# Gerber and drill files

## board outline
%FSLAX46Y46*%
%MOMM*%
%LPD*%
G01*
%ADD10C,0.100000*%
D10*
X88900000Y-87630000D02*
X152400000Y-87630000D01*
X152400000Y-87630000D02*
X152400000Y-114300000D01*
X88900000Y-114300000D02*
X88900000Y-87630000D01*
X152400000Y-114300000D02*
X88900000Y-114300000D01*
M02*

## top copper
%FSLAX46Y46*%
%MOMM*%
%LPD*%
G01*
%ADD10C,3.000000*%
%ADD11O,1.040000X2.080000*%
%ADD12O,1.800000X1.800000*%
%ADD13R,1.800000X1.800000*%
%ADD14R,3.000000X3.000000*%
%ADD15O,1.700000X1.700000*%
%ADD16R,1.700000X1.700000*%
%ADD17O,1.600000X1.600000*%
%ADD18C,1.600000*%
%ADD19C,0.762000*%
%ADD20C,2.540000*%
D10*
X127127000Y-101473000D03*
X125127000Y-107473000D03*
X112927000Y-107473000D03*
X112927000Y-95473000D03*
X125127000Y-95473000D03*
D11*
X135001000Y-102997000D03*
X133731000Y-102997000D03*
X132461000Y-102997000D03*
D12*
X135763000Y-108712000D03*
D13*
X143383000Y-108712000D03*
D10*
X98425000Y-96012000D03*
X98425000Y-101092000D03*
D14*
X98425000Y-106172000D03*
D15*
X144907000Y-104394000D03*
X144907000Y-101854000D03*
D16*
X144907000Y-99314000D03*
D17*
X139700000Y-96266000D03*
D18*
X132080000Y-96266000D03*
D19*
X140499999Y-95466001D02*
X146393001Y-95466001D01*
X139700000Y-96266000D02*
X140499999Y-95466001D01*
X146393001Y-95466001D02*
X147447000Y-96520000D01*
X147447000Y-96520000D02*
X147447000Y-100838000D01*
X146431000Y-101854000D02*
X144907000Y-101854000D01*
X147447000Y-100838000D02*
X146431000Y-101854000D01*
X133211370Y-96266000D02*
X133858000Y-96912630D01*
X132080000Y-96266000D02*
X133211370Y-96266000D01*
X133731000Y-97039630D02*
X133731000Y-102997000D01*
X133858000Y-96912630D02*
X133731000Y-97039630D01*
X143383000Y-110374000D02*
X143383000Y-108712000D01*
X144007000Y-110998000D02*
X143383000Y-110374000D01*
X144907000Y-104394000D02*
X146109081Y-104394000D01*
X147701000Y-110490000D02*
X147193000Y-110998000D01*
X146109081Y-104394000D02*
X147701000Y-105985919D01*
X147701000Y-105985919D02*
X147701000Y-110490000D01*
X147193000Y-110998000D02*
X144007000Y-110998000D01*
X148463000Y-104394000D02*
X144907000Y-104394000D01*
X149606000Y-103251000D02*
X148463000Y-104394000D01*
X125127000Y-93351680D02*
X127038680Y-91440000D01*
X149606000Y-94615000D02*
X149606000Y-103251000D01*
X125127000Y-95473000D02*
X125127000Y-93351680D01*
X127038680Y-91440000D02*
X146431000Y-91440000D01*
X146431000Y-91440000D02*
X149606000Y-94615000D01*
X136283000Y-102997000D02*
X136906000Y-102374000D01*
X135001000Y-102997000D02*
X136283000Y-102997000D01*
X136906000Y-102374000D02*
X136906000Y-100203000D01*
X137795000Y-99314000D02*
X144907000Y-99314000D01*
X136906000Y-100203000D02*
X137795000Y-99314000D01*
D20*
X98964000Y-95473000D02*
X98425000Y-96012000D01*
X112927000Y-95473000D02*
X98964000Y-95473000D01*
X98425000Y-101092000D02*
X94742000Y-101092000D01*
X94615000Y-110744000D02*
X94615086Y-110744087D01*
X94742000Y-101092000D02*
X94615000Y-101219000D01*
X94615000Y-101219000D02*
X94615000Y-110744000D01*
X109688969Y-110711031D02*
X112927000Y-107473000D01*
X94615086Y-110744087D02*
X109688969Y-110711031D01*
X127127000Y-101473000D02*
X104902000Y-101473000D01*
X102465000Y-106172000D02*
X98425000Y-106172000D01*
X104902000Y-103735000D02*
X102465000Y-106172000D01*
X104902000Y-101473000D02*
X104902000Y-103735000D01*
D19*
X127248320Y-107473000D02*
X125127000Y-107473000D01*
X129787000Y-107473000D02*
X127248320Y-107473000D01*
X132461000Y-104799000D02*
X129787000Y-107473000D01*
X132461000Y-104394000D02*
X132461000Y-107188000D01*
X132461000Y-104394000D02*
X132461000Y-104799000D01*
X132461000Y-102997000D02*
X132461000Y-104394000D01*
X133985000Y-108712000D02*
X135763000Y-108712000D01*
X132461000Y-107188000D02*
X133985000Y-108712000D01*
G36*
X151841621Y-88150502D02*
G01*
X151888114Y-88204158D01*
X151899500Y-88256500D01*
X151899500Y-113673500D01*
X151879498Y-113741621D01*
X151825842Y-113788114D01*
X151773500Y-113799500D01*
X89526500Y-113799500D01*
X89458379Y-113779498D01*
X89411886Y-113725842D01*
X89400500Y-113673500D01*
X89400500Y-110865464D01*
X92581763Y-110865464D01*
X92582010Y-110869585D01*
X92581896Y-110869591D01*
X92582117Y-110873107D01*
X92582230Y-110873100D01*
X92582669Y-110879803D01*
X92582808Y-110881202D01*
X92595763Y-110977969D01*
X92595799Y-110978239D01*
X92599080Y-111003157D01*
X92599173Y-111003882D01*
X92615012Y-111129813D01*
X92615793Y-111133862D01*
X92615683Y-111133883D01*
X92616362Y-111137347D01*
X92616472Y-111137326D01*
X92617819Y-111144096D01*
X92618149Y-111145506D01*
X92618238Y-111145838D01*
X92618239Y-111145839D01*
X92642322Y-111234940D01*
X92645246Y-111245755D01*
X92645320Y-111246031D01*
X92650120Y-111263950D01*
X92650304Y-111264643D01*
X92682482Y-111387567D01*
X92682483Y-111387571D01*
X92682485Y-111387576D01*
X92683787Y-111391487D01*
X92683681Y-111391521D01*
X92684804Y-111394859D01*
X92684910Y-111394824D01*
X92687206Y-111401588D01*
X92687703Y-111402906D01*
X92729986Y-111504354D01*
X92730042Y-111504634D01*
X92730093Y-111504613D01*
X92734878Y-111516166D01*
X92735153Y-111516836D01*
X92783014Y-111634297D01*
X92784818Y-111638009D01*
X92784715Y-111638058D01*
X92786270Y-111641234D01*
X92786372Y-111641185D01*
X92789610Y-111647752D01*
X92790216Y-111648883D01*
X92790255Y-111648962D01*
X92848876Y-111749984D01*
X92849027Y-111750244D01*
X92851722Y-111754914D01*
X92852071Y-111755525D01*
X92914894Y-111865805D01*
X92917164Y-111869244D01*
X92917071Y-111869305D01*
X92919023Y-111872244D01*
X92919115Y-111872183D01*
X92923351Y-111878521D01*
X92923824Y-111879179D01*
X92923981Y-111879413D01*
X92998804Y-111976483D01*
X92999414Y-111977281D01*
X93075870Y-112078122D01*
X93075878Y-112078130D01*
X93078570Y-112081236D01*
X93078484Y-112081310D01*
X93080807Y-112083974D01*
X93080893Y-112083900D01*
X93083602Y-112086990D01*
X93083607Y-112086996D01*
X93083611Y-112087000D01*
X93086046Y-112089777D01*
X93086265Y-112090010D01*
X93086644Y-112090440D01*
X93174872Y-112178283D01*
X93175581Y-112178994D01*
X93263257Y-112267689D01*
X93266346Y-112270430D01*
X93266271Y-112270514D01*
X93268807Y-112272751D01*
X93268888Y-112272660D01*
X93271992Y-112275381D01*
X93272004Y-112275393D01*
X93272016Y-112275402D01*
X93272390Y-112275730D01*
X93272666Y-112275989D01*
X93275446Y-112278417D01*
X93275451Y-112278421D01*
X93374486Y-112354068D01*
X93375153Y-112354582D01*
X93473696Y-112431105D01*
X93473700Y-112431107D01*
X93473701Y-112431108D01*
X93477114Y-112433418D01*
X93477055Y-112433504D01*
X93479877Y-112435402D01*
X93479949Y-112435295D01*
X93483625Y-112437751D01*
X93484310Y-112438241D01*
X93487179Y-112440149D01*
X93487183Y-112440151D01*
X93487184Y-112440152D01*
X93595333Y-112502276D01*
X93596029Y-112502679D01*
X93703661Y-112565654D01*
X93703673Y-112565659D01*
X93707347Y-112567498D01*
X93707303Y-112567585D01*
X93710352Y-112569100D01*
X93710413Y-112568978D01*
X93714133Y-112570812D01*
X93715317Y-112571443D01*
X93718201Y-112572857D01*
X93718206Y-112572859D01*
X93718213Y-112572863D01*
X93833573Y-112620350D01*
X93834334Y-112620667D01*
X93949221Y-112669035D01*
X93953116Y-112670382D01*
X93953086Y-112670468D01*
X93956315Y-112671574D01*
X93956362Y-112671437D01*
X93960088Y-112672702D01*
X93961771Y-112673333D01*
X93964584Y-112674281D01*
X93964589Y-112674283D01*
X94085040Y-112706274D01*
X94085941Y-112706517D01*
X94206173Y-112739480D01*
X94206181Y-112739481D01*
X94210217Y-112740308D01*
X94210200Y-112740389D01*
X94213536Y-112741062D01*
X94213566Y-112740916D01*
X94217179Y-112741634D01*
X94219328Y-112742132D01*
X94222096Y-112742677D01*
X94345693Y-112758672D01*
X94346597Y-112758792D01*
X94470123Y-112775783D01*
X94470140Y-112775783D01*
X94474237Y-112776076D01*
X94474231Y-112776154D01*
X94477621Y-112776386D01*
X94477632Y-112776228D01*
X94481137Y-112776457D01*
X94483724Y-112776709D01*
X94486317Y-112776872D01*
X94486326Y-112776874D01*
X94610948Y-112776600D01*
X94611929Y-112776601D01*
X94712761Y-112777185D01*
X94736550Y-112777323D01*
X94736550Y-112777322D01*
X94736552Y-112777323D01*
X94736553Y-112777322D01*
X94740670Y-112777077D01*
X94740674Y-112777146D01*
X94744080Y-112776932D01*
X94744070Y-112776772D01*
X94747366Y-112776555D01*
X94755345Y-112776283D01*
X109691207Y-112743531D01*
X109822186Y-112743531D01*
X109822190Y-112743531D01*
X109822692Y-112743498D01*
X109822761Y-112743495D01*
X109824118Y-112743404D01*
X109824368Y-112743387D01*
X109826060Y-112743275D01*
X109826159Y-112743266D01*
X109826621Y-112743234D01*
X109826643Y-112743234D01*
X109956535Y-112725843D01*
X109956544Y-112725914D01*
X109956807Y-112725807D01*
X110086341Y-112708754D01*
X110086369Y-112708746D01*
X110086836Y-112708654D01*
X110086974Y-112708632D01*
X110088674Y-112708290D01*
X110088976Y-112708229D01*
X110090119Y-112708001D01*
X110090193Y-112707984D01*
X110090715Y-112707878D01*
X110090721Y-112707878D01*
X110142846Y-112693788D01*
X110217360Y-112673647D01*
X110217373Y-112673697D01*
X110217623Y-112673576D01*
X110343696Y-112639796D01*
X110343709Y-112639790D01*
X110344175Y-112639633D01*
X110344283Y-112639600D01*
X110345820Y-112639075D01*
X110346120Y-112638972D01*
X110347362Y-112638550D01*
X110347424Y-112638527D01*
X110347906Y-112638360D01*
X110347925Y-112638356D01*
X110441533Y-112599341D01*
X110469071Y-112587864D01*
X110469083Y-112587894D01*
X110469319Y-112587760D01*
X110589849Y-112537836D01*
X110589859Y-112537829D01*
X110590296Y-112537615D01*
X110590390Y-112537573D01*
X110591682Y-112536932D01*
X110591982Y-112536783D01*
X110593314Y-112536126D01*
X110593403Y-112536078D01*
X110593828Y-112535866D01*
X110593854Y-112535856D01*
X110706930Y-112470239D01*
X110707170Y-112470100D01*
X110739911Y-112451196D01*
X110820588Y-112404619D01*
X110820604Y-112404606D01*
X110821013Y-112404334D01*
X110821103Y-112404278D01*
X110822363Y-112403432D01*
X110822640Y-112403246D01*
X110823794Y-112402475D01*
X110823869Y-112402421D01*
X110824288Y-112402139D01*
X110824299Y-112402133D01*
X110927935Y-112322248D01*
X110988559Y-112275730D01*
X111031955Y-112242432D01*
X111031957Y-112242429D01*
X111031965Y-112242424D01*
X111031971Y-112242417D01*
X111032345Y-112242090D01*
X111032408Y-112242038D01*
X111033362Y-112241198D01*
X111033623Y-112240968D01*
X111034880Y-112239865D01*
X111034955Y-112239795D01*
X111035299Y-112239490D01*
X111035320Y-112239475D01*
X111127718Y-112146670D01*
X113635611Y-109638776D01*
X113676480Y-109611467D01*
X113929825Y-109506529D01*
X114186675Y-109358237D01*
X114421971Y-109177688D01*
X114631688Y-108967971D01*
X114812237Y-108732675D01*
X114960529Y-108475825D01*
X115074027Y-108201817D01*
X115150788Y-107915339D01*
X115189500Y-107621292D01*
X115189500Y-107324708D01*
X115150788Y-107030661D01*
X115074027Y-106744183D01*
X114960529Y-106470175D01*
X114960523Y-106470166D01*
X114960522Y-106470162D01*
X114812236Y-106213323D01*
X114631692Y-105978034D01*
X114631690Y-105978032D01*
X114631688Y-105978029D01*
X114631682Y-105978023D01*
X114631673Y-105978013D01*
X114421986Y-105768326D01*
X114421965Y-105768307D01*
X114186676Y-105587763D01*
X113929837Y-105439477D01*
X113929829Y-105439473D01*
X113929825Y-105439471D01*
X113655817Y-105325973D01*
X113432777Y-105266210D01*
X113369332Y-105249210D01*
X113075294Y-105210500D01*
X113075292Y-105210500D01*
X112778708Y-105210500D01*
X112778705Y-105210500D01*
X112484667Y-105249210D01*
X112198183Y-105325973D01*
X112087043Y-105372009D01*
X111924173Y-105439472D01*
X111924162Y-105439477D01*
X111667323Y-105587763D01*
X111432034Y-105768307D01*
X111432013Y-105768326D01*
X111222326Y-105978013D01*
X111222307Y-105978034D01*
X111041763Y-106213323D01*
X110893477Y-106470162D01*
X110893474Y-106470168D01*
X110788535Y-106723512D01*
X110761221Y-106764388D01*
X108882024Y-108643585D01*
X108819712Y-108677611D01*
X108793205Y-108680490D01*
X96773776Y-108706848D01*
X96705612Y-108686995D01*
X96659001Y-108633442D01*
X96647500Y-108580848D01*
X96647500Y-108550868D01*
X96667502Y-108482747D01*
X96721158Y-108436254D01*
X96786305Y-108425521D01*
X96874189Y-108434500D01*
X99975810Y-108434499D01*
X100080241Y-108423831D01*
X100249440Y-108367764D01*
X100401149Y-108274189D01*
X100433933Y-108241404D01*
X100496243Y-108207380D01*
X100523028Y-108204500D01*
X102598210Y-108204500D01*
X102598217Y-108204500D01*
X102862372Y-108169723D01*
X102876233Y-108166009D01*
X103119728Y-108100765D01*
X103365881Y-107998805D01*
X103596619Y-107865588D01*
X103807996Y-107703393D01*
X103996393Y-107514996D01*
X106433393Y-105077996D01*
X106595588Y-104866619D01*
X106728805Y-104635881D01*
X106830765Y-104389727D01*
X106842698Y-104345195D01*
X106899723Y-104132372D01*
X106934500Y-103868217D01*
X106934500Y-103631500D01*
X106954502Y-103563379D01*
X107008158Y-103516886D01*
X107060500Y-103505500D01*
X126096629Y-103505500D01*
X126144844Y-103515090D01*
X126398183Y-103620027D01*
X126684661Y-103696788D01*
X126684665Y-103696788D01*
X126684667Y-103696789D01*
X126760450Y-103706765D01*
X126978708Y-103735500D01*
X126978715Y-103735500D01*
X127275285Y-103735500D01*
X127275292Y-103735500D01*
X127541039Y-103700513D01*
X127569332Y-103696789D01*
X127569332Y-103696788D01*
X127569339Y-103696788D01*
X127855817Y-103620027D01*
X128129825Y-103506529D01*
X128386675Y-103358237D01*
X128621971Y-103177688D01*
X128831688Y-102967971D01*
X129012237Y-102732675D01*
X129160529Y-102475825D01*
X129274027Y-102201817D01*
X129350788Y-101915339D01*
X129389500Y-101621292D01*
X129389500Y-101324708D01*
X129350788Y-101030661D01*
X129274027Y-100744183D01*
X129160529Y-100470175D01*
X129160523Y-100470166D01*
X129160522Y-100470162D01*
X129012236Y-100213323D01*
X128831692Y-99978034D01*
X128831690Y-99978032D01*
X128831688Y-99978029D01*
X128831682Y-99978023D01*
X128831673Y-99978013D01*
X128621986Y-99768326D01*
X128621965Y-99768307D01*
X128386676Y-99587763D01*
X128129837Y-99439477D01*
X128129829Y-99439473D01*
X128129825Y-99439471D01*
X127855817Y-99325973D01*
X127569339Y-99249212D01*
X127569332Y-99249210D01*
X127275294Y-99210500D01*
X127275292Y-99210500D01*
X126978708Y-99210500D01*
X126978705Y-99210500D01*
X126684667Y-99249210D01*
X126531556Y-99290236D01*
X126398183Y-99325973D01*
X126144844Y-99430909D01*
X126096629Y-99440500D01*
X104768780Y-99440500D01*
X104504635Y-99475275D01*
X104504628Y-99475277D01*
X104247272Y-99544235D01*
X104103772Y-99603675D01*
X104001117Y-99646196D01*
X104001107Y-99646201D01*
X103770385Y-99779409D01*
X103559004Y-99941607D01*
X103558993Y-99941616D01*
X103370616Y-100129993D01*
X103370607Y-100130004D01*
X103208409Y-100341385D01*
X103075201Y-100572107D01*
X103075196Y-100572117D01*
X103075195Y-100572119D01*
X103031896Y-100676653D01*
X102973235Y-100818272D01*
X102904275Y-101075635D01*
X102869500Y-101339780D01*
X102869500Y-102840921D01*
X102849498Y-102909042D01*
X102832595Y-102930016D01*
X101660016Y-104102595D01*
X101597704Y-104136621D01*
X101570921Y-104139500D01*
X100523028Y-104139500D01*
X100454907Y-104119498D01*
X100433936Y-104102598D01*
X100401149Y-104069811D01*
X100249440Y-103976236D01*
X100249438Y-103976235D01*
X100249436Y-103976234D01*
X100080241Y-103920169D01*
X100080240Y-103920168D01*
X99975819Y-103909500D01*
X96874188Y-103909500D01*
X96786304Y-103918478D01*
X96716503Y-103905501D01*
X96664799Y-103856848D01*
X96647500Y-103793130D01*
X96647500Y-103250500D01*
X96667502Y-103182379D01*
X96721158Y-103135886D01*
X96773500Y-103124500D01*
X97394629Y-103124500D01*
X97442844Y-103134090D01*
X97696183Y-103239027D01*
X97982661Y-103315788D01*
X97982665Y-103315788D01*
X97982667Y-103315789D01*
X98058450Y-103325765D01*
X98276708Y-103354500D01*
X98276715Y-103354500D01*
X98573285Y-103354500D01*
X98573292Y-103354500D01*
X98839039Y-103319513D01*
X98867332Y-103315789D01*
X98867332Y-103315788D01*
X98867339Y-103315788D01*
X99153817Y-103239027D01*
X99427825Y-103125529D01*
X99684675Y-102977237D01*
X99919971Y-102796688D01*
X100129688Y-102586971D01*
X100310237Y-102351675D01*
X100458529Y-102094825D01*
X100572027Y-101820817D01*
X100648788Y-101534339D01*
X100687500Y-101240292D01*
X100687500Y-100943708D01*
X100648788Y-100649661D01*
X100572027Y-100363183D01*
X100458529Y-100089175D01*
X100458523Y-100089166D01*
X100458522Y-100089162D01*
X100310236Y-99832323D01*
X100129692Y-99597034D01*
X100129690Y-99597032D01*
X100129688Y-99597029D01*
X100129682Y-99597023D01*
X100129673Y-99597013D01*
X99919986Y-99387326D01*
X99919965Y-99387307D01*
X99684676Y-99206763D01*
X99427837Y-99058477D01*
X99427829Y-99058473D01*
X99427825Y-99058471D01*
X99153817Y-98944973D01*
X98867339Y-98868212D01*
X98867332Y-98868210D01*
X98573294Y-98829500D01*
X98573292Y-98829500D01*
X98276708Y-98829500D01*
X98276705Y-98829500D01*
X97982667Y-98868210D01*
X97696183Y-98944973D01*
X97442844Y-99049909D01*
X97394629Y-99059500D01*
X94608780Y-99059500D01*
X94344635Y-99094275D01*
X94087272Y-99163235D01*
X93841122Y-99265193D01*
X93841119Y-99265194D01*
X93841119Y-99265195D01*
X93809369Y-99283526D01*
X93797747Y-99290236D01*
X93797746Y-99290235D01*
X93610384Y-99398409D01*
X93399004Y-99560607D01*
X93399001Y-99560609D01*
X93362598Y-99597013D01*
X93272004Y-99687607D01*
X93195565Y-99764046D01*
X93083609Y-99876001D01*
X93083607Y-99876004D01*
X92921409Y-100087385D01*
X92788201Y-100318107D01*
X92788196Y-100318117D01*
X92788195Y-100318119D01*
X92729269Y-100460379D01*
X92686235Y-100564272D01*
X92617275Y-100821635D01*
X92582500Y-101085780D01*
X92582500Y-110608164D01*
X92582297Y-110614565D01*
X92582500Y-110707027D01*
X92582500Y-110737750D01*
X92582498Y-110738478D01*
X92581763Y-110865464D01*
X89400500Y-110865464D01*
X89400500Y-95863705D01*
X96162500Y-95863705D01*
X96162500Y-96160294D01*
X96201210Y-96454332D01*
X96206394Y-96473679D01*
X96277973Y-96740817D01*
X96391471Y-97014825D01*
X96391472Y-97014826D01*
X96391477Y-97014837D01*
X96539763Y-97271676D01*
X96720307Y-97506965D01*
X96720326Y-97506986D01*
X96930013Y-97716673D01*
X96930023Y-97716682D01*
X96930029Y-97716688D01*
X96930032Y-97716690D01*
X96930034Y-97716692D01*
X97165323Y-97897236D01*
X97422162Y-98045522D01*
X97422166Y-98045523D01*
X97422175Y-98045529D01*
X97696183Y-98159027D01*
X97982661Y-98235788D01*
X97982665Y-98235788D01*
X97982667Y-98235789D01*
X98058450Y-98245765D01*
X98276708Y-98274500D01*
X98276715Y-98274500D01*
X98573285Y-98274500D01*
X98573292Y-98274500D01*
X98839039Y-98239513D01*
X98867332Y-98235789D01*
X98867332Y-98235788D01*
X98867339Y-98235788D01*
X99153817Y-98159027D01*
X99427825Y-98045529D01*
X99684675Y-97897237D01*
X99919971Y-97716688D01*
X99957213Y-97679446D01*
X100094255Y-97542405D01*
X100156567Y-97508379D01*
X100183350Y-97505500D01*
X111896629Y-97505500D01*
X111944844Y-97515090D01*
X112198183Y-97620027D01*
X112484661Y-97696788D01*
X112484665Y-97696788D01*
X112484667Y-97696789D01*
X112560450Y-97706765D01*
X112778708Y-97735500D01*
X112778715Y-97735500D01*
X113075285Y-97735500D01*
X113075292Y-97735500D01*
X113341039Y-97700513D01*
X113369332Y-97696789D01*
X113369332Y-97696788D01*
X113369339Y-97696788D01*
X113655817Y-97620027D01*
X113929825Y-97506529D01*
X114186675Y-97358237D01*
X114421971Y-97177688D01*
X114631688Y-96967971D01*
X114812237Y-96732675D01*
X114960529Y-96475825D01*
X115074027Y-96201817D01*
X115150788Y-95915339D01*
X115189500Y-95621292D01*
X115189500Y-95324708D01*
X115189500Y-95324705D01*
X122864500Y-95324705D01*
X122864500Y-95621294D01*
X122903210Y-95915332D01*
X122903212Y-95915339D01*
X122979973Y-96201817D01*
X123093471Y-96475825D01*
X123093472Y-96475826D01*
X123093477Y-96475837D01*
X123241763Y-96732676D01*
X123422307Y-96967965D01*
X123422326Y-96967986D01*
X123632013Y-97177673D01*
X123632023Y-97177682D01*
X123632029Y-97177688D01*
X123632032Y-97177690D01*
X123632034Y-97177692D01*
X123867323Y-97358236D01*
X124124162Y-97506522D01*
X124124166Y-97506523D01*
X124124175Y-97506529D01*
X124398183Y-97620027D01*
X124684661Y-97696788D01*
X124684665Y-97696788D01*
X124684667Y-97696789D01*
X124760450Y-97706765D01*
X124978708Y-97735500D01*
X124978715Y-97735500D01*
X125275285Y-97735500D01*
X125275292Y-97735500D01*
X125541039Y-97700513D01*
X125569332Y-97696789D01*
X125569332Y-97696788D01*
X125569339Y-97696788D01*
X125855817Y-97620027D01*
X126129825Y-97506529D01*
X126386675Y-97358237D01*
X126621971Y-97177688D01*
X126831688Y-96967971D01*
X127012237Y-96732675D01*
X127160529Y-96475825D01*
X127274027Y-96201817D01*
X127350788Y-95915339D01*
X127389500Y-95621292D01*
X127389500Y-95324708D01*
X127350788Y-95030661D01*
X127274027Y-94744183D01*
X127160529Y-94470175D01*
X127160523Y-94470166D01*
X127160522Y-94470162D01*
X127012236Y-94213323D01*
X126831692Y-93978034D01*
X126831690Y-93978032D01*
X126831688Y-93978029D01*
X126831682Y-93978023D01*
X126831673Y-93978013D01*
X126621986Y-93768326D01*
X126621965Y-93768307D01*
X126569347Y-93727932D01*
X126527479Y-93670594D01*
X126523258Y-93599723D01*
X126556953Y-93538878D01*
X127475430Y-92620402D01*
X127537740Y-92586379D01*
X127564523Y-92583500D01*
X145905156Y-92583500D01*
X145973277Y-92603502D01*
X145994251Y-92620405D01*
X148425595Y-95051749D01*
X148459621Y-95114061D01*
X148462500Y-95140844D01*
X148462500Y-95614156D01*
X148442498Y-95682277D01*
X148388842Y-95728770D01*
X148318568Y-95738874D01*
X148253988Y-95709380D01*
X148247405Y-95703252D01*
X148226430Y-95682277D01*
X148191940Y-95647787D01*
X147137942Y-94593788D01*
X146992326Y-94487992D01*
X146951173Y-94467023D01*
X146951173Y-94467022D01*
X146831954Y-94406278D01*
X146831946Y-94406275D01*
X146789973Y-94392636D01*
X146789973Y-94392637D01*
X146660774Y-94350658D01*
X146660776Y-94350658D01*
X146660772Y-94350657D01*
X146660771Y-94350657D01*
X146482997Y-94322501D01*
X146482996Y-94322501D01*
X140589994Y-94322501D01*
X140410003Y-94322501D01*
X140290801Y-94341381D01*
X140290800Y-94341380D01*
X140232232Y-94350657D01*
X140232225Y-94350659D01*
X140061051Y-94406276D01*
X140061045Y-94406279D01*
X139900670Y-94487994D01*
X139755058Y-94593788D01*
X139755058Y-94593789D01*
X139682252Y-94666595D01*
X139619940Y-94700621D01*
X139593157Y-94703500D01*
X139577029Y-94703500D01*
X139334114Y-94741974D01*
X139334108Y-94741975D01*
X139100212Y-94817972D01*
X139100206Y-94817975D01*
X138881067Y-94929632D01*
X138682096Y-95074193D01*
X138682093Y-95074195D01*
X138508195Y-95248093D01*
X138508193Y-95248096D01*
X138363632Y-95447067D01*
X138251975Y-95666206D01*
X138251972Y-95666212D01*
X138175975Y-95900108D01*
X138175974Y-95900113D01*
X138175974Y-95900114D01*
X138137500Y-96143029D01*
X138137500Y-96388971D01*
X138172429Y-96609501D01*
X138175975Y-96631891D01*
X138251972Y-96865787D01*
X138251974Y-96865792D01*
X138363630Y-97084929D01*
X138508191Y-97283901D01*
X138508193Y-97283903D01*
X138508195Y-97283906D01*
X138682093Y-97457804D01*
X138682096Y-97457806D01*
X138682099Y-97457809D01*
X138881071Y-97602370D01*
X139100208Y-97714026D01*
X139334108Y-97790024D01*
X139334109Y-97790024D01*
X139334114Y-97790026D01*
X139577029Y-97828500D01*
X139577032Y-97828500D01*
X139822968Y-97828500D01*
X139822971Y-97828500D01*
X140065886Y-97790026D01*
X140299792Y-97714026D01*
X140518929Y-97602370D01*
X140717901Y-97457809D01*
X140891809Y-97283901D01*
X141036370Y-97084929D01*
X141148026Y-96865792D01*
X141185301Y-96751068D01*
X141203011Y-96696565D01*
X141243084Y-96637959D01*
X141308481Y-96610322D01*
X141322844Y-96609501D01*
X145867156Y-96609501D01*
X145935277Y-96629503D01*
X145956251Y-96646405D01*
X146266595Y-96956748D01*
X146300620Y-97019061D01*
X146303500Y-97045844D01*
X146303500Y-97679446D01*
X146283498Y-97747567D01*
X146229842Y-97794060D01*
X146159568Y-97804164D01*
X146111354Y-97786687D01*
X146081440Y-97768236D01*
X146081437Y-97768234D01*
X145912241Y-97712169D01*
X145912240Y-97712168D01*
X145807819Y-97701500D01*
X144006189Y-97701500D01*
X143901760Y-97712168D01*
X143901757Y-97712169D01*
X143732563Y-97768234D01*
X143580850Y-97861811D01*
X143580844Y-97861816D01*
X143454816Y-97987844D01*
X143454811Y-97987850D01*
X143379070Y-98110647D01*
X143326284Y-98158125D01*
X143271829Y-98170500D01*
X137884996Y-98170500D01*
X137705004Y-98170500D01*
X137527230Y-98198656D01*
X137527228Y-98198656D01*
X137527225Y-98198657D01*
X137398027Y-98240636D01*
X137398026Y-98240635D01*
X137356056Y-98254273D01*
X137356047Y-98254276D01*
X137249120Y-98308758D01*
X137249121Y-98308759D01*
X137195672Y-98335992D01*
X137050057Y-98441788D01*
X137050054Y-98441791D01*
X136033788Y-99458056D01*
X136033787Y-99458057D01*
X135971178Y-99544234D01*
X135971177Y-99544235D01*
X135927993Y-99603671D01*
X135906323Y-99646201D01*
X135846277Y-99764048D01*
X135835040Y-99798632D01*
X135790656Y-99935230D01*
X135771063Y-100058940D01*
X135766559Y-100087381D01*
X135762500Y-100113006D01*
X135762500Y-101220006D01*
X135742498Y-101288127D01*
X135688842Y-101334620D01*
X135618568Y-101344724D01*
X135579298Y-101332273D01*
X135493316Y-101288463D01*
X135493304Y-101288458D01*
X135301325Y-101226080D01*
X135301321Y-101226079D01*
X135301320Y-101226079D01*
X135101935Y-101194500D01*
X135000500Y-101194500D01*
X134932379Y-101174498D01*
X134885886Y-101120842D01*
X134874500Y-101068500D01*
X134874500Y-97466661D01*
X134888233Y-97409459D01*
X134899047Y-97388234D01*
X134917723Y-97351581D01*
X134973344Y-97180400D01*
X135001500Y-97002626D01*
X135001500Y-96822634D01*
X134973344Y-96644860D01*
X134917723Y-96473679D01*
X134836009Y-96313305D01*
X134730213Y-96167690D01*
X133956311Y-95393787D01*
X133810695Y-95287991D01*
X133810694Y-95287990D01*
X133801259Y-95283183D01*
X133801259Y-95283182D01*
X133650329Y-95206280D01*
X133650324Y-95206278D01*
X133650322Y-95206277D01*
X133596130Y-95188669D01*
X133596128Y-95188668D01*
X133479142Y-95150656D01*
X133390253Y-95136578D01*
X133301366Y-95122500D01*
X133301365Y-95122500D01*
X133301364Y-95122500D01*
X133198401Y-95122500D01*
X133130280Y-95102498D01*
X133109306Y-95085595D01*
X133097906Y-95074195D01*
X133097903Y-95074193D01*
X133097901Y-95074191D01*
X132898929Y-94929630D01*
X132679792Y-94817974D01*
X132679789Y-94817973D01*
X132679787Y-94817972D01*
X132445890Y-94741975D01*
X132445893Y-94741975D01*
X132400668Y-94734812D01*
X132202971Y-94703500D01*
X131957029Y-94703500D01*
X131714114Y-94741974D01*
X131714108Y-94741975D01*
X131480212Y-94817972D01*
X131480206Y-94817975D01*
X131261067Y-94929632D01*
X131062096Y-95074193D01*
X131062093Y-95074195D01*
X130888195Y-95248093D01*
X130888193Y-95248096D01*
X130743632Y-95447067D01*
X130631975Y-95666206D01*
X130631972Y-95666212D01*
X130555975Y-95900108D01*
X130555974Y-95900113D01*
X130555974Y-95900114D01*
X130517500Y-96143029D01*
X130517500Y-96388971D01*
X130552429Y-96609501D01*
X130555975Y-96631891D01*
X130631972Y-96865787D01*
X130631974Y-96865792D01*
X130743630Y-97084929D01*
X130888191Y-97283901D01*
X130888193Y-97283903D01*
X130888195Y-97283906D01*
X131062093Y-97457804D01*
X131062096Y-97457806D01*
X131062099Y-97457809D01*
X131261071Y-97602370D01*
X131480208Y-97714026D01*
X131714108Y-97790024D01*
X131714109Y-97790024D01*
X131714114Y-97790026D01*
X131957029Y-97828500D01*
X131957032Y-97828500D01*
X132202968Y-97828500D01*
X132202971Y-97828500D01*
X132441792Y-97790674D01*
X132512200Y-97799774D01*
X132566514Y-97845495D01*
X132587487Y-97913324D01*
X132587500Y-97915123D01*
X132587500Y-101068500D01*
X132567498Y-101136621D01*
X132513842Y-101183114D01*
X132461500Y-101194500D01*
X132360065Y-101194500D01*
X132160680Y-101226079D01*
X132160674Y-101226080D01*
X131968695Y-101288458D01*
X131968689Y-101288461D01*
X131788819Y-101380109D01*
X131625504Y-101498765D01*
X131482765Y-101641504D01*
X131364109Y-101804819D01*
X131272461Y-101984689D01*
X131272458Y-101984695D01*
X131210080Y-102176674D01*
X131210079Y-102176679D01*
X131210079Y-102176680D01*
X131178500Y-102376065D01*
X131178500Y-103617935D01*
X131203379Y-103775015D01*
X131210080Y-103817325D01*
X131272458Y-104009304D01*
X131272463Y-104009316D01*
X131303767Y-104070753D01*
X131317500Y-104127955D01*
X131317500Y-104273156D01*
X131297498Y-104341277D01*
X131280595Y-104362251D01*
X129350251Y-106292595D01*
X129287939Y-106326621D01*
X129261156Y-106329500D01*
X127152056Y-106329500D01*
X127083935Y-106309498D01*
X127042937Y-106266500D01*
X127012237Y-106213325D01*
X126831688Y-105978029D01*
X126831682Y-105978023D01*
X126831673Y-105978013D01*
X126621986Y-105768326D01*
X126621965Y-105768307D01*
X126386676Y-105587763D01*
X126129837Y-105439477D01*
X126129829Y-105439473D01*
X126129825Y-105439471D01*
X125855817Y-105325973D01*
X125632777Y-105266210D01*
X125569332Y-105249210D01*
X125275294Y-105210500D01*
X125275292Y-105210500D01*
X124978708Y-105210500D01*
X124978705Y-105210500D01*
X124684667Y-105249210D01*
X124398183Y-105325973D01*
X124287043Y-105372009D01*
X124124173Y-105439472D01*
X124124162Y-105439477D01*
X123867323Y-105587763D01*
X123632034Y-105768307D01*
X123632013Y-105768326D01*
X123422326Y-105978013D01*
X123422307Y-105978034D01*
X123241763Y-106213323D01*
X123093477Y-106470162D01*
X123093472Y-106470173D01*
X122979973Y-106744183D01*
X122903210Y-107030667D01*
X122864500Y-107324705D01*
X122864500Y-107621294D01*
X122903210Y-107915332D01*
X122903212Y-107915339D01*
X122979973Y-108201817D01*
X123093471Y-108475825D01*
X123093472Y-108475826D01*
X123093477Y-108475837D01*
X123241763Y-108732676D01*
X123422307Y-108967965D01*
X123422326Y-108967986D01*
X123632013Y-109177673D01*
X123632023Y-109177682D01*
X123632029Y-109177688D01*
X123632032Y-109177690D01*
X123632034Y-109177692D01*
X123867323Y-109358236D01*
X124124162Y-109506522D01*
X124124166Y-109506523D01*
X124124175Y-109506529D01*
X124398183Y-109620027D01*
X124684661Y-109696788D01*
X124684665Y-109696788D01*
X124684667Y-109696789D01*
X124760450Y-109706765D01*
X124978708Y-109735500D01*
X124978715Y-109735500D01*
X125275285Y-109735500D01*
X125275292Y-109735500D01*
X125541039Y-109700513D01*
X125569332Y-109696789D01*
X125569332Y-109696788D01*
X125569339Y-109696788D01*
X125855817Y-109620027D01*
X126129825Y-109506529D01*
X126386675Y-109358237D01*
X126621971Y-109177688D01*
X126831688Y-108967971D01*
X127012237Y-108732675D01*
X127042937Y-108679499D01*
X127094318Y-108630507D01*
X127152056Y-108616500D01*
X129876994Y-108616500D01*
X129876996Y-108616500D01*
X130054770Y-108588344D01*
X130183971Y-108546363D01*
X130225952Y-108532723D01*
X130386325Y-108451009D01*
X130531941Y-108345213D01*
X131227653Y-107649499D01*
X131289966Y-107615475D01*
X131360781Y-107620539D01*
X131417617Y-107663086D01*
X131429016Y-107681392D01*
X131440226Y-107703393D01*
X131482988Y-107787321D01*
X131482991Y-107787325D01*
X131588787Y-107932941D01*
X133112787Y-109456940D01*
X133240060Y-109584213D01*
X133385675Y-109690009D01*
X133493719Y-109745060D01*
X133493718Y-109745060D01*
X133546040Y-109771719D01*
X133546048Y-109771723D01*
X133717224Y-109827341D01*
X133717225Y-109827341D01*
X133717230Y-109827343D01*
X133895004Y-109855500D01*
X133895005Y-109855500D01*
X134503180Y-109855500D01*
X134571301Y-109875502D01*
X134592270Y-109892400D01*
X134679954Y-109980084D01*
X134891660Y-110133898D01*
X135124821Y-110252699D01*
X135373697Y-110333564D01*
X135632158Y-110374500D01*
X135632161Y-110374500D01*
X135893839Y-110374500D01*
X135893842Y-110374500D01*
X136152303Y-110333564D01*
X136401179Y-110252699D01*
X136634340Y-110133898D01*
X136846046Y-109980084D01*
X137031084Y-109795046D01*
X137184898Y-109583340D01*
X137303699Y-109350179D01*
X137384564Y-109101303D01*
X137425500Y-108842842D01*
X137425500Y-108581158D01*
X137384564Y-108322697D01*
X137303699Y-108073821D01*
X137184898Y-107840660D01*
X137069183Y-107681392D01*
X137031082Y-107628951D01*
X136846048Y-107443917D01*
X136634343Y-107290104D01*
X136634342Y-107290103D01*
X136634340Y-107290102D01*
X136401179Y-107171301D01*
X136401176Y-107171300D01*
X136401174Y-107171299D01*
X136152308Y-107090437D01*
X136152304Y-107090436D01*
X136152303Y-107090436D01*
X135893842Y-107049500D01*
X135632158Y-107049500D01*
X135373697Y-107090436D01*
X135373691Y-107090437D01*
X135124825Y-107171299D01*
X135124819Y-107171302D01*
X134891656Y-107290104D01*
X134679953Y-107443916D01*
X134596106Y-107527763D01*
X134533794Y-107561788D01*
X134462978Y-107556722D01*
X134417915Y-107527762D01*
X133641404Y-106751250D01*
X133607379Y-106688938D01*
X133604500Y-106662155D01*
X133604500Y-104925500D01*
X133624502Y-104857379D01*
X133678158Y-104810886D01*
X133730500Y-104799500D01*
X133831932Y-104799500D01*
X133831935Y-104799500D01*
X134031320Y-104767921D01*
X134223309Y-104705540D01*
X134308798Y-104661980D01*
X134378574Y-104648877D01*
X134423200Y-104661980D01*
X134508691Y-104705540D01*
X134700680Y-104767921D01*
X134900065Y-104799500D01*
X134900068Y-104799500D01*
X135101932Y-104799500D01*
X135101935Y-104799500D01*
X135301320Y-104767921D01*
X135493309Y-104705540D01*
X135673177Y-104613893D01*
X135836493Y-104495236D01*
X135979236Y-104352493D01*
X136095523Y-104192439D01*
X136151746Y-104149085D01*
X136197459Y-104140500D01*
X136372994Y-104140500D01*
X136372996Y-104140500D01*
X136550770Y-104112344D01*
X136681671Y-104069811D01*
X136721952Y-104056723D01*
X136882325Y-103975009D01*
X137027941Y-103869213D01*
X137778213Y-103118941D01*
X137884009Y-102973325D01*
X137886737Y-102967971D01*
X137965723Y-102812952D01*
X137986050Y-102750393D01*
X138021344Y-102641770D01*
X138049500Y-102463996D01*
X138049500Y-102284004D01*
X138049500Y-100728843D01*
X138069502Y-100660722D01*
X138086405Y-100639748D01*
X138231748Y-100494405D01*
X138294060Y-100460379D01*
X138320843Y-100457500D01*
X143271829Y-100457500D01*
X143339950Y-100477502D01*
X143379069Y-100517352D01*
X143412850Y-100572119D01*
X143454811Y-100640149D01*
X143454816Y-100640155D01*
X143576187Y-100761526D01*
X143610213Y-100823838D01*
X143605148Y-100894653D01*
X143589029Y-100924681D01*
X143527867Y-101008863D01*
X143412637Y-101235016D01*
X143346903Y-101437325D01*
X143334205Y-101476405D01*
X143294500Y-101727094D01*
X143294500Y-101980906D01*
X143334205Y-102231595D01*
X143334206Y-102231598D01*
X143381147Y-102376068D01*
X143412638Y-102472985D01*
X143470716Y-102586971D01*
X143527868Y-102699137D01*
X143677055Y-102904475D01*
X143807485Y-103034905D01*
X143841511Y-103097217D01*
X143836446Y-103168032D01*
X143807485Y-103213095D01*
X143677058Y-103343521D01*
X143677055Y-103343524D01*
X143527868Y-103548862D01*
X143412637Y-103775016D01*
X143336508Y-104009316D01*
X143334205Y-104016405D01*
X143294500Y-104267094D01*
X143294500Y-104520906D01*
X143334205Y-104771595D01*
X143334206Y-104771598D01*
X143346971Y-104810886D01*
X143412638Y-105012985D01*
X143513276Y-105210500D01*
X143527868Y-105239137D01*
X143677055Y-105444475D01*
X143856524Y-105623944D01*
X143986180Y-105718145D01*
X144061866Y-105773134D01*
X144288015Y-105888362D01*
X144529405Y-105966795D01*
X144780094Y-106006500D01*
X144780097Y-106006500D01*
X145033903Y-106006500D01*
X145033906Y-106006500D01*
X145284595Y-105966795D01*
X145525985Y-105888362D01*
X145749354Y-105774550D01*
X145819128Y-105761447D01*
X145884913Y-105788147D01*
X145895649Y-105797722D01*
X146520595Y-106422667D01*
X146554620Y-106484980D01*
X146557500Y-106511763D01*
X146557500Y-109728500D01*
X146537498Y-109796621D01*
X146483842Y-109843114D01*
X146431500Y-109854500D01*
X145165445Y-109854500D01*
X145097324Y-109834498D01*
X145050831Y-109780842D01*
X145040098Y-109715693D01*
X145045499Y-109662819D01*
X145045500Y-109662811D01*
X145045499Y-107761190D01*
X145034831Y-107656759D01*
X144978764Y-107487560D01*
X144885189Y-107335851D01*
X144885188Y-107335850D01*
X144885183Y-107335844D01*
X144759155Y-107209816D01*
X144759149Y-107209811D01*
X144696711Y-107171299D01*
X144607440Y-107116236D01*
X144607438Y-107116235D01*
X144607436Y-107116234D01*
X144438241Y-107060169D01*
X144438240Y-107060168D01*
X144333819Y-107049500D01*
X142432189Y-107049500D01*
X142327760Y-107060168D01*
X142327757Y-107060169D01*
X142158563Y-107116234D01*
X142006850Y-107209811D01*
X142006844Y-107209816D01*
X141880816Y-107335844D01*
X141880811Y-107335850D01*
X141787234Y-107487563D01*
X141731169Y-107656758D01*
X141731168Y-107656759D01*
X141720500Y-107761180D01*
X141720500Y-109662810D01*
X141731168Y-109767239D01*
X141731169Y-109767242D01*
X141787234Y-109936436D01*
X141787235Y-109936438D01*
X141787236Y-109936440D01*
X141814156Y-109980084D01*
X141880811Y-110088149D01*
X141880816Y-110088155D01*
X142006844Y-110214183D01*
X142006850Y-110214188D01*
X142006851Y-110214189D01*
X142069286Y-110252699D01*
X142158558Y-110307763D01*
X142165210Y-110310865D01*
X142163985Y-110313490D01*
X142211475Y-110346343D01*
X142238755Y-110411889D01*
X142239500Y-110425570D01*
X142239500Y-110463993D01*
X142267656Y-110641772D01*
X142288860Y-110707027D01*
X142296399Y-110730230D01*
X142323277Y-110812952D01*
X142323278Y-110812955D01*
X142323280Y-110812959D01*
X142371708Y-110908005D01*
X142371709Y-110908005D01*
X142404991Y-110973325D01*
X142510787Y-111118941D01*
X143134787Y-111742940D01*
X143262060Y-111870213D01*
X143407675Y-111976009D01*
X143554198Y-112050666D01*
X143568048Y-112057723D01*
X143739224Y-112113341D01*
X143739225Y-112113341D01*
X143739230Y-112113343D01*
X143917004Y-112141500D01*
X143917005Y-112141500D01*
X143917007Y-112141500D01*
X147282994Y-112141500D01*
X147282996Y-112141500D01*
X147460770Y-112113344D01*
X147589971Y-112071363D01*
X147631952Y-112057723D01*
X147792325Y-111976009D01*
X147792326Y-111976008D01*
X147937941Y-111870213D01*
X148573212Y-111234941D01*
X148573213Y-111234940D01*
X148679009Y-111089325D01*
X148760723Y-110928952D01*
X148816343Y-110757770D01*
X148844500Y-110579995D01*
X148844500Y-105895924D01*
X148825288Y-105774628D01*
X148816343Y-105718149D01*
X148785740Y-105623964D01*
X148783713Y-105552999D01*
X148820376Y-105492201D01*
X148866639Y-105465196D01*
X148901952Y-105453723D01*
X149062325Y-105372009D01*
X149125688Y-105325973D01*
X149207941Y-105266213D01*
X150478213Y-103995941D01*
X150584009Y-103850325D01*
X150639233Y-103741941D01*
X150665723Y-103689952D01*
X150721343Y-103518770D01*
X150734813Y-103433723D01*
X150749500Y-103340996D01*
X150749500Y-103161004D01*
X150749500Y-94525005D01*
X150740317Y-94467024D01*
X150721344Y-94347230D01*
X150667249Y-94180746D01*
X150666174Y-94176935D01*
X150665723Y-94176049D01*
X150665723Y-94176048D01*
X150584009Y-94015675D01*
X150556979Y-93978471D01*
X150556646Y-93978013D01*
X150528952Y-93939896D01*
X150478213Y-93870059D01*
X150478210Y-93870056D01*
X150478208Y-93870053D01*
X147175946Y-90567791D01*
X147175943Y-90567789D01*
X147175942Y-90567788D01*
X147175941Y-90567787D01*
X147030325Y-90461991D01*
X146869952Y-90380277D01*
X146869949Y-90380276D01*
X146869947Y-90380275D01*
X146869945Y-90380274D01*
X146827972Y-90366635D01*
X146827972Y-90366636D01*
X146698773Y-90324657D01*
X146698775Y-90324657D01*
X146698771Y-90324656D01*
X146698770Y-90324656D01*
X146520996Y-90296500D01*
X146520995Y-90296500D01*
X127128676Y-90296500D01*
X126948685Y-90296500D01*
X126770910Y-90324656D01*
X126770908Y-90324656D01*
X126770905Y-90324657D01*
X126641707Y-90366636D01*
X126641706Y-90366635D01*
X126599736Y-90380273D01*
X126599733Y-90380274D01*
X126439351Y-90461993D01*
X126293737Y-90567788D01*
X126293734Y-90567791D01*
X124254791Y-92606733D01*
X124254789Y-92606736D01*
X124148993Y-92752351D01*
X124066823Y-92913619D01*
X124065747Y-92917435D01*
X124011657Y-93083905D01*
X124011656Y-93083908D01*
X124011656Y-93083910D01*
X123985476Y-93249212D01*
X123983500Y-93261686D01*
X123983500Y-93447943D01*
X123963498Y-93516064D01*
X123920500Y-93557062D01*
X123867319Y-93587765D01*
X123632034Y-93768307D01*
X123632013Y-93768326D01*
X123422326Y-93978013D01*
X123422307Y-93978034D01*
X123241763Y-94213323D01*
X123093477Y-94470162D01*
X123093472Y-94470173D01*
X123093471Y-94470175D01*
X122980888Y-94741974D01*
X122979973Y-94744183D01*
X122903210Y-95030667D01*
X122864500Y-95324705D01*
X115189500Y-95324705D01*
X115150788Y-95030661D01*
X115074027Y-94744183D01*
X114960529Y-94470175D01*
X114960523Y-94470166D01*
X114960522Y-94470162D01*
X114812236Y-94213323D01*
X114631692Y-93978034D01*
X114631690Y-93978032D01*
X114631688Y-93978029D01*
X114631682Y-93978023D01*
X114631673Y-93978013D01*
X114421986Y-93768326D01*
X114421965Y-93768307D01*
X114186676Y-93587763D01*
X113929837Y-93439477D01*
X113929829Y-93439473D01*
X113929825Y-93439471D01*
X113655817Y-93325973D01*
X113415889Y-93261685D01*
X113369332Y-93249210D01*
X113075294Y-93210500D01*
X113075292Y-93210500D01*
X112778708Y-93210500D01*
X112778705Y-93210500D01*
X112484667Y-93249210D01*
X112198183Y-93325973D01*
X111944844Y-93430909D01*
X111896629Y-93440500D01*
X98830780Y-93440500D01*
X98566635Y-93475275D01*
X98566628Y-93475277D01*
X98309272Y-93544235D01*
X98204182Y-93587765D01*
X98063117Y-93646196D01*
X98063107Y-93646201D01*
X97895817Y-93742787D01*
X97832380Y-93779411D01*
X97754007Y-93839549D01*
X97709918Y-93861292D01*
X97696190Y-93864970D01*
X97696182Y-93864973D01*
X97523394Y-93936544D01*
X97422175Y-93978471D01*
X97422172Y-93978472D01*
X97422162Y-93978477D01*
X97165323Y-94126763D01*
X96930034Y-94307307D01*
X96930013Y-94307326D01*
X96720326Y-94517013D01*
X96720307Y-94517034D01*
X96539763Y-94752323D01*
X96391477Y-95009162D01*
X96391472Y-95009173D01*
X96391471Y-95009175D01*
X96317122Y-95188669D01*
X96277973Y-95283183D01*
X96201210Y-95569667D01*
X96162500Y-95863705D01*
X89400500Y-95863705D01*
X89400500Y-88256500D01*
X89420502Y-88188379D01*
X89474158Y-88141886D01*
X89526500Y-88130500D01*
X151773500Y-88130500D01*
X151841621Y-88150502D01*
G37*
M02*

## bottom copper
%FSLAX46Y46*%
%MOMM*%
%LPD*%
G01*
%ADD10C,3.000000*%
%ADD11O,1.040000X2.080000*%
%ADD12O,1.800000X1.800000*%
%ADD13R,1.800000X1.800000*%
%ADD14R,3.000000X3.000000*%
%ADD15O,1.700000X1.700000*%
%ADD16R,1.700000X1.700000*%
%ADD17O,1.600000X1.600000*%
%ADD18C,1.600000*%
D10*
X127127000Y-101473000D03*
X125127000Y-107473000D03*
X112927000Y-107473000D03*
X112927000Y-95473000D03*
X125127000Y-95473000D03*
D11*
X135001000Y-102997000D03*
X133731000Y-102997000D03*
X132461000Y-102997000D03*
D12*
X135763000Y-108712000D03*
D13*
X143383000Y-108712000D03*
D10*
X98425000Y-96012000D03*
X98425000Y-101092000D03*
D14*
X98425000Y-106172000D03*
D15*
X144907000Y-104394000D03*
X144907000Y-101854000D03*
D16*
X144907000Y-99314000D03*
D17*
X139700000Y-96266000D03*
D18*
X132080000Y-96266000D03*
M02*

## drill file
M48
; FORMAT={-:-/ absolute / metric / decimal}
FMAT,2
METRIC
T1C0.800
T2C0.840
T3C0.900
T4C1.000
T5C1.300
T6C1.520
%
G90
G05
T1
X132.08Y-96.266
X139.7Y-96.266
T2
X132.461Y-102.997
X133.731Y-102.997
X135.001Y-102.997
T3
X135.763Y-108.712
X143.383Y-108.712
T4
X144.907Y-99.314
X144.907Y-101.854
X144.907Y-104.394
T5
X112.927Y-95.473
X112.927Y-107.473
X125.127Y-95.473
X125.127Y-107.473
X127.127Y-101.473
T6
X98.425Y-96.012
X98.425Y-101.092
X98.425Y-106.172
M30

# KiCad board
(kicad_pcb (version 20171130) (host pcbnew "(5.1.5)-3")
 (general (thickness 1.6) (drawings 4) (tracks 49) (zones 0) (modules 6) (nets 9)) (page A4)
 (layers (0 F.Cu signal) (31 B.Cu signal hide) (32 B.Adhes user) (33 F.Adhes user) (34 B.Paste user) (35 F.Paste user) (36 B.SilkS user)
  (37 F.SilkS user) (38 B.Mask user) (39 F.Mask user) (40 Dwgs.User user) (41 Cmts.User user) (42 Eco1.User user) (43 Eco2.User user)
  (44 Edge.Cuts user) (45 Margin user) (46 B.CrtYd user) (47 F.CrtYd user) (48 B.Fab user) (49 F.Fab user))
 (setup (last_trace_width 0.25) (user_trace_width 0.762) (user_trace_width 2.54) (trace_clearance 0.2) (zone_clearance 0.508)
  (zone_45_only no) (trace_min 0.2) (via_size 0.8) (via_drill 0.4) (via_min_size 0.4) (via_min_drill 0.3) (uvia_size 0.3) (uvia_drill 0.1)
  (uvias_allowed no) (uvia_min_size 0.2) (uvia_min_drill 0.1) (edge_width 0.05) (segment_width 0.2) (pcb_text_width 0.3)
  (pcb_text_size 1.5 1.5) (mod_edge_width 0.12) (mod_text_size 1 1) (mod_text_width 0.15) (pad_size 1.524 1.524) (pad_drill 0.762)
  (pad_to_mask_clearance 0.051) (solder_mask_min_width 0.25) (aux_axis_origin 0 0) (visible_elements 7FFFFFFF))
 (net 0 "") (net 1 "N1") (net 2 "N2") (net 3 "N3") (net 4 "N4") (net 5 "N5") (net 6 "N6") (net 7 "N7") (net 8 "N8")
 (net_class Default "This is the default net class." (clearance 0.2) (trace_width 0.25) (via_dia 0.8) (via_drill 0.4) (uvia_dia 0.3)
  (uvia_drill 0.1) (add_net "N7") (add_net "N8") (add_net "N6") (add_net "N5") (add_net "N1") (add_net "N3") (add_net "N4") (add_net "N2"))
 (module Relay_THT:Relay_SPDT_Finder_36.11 (layer F.Cu) (at 127.127 101.473 180)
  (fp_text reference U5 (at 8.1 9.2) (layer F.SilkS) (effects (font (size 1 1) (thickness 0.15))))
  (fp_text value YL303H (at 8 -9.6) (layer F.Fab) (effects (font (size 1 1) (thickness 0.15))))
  (pad 11 thru_hole circle (at 0 0 180) (size 3 3) (drill 1.3) (layers *.Cu *.Mask) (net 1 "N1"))
  (pad A2 thru_hole circle (at 2 -6 180) (size 3 3) (drill 1.3) (layers *.Cu *.Mask) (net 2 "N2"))
  (pad 12 thru_hole circle (at 14.2 -6 180) (size 3 3) (drill 1.3) (layers *.Cu *.Mask) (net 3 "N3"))
  (pad 14 thru_hole circle (at 14.2 6 180) (size 3 3) (drill 1.3) (layers *.Cu *.Mask) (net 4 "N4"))
  (pad A1 thru_hole circle (at 2 6 180) (size 3 3) (drill 1.3) (layers *.Cu *.Mask) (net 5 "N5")))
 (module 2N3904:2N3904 (layer F.Cu) (at 133.731 102.997 180)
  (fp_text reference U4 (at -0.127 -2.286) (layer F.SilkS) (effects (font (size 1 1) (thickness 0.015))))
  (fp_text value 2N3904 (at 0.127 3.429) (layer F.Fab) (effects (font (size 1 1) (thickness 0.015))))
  (pad 1 thru_hole oval (at -1.27 0 180) (size 1.04 2.08) (drill 0.84) (layers *.Cu *.Mask) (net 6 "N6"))
  (pad 2 thru_hole oval (at 0 0 180) (size 1.04 2.08) (drill 0.84) (layers *.Cu *.Mask) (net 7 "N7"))
  (pad 3 thru_hole oval (at 1.27 0 180) (size 1.04 2.08) (drill 0.84) (layers *.Cu *.Mask) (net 2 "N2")))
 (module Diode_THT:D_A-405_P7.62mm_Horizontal (layer F.Cu) (at 143.383 108.712 180)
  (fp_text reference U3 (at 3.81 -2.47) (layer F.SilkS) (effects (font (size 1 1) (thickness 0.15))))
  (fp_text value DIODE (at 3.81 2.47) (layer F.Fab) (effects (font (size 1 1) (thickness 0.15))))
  (pad 2 thru_hole oval (at 7.62 0 180) (size 1.8 1.8) (drill 0.9) (layers *.Cu *.Mask) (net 2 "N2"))
  (pad 1 thru_hole rect (at 0 0 180) (size 1.8 1.8) (drill 0.9) (layers *.Cu *.Mask) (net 5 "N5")))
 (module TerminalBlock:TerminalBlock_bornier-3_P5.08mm (layer F.Cu) (at 98.425 106.172 90)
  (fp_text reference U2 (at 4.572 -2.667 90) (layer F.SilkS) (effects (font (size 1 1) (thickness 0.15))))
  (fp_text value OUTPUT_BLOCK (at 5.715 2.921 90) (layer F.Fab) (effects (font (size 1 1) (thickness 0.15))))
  (pad 3 thru_hole circle (at 10.16 0 90) (size 3 3) (drill 1.52) (layers *.Cu *.Mask) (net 4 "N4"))
  (pad 2 thru_hole circle (at 5.08 0 90) (size 3 3) (drill 1.52) (layers *.Cu *.Mask) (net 3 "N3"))
  (pad 1 thru_hole rect (at 0 0 90) (size 3 3) (drill 1.52) (layers *.Cu *.Mask) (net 1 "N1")))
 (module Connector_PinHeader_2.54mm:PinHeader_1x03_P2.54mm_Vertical (layer F.Cu) (at 144.907 99.314)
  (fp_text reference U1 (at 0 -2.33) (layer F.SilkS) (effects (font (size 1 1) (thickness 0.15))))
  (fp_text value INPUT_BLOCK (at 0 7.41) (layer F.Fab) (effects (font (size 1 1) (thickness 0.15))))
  (pad 3 thru_hole oval (at 0 5.08) (size 1.7 1.7) (drill 1) (layers *.Cu *.Mask) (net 5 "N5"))
  (pad 2 thru_hole oval (at 0 2.54) (size 1.7 1.7) (drill 1) (layers *.Cu *.Mask) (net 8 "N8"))
  (pad 1 thru_hole rect (at 0 0) (size 1.7 1.7) (drill 1) (layers *.Cu *.Mask) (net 6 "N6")))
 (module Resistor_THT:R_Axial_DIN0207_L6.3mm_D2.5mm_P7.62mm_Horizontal (layer F.Cu) (at 132.08 96.266)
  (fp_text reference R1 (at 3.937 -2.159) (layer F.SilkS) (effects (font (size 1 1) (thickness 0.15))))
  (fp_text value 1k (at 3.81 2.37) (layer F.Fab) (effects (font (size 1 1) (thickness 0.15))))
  (pad 2 thru_hole oval (at 7.62 0) (size 1.6 1.6) (drill 0.8) (layers *.Cu *.Mask) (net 8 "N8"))
  (pad 1 thru_hole circle (at 0 0) (size 1.6 1.6) (drill 0.8) (layers *.Cu *.Mask) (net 7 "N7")))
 (gr_line (start 88.9 87.63) (end 152.4 87.63) (layer Edge.Cuts) (width 0.1))
 (gr_line (start 152.4 87.63) (end 152.4 114.3) (layer Edge.Cuts) (width 0.1))
 (gr_line (start 88.9 114.3) (end 88.9 87.63) (layer Edge.Cuts) (width 0.1))
 (gr_line (start 152.4 114.3) (end 88.9 114.3) (layer Edge.Cuts) (width 0.1))
 (segment (start 140.499999 95.466001) (end 146.393001 95.466001) (width 0.762) (layer F.Cu) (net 8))
 (segment (start 139.7 96.266) (end 140.499999 95.466001) (width 0.762) (layer F.Cu) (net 8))
 (segment (start 146.393001 95.466001) (end 147.447 96.52) (width 0.762) (layer F.Cu) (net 8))
 (segment (start 147.447 96.52) (end 147.447 100.838) (width 0.762) (layer F.Cu) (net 8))
 (segment (start 146.431 101.854) (end 144.907 101.854) (width 0.762) (layer F.Cu) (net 8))
 (segment (start 147.447 100.838) (end 146.431 101.854) (width 0.762) (layer F.Cu) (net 8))
 (segment (start 133.21137 96.266) (end 133.858 96.91263) (width 0.762) (layer F.Cu) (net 7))
 (segment (start 132.08 96.266) (end 133.21137 96.266) (width 0.762) (layer F.Cu) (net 7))
 (segment (start 133.731 97.03963) (end 133.731 102.997) (width 0.762) (layer F.Cu) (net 7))
 (segment (start 133.858 96.91263) (end 133.731 97.03963) (width 0.762) (layer F.Cu) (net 7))
 (segment (start 143.383 110.374) (end 143.383 108.712) (width 0.762) (layer F.Cu) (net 5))
 (segment (start 144.007 110.998) (end 143.383 110.374) (width 0.762) (layer F.Cu) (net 5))
 (segment (start 144.907 104.394) (end 146.109081 104.394) (width 0.762) (layer F.Cu) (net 5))
 (segment (start 147.701 110.49) (end 147.193 110.998) (width 0.762) (layer F.Cu) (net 5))
 (segment (start 146.109081 104.394) (end 147.701 105.985919) (width 0.762) (layer F.Cu) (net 5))
 (segment (start 147.701 105.985919) (end 147.701 110.49) (width 0.762) (layer F.Cu) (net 5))
 (segment (start 147.193 110.998) (end 144.007 110.998) (width 0.762) (layer F.Cu) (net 5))
 (segment (start 148.463 104.394) (end 144.907 104.394) (width 0.762) (layer F.Cu) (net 5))
 (segment (start 149.606 103.251) (end 148.463 104.394) (width 0.762) (layer F.Cu) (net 5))
 (segment (start 125.127 93.35168) (end 127.03868 91.44) (width 0.762) (layer F.Cu) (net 5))
 (segment (start 149.606 94.615) (end 149.606 103.251) (width 0.762) (layer F.Cu) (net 5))
 (segment (start 125.127 95.473) (end 125.127 93.35168) (width 0.762) (layer F.Cu) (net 5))
 (segment (start 127.03868 91.44) (end 146.431 91.44) (width 0.762) (layer F.Cu) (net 5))
 (segment (start 146.431 91.44) (end 149.606 94.615) (width 0.762) (layer F.Cu) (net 5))
 (segment (start 136.283 102.997) (end 136.906 102.374) (width 0.762) (layer F.Cu) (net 6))
 (segment (start 135.001 102.997) (end 136.283 102.997) (width 0.762) (layer F.Cu) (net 6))
 (segment (start 136.906 102.374) (end 136.906 100.203) (width 0.762) (layer F.Cu) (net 6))
 (segment (start 137.795 99.314) (end 144.907 99.314) (width 0.762) (layer F.Cu) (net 6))
 (segment (start 136.906 100.203) (end 137.795 99.314) (width 0.762) (layer F.Cu) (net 6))
 (segment (start 98.964 95.473) (end 98.425 96.012) (width 2.54) (layer F.Cu) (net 4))
 (segment (start 112.927 95.473) (end 98.964 95.473) (width 2.54) (layer F.Cu) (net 4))
 (segment (start 98.425 101.092) (end 94.742 101.092) (width 2.54) (layer F.Cu) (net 3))
 (segment (start 94.615 110.744) (end 94.615086 110.744087) (width 2.54) (layer F.Cu) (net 3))
 (segment (start 94.742 101.092) (end 94.615 101.219) (width 2.54) (layer F.Cu) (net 3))
 (segment (start 94.615 101.219) (end 94.615 110.744) (width 2.54) (layer F.Cu) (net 3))
 (segment (start 109.688969 110.711031) (end 112.927 107.473) (width 2.54) (layer F.Cu) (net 3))
 (segment (start 94.615086 110.744087) (end 109.688969 110.711031) (width 2.54) (layer F.Cu) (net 3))
 (segment (start 127.127 101.473) (end 104.902 101.473) (width 2.54) (layer F.Cu) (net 1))
 (segment (start 102.465 106.172) (end 98.425 106.172) (width 2.54) (layer F.Cu) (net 1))
 (segment (start 104.902 103.735) (end 102.465 106.172) (width 2.54) (layer F.Cu) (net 1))
 (segment (start 104.902 101.473) (end 104.902 103.735) (width 2.54) (layer F.Cu) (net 1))
 (segment (start 127.24832 107.473) (end 125.127 107.473) (width 0.762) (layer F.Cu) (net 2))
 (segment (start 129.787 107.473) (end 127.24832 107.473) (width 0.762) (layer F.Cu) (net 2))
 (segment (start 132.461 104.799) (end 129.787 107.473) (width 0.762) (layer F.Cu) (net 2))
 (segment (start 132.461 104.394) (end 132.461 107.188) (width 0.762) (layer F.Cu) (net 2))
 (segment (start 132.461 104.394) (end 132.461 104.799) (width 0.762) (layer F.Cu) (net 2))
 (segment (start 132.461 102.997) (end 132.461 104.394) (width 0.762) (layer F.Cu) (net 2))
 (segment (start 133.985 108.712) (end 135.763 108.712) (width 0.762) (layer F.Cu) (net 2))
 (segment (start 132.461 107.188) (end 133.985 108.712) (width 0.762) (layer F.Cu) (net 2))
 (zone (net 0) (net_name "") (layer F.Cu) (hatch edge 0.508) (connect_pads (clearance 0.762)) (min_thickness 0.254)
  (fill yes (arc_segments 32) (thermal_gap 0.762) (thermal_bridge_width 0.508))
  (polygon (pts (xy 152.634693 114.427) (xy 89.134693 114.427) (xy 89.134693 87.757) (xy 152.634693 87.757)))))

